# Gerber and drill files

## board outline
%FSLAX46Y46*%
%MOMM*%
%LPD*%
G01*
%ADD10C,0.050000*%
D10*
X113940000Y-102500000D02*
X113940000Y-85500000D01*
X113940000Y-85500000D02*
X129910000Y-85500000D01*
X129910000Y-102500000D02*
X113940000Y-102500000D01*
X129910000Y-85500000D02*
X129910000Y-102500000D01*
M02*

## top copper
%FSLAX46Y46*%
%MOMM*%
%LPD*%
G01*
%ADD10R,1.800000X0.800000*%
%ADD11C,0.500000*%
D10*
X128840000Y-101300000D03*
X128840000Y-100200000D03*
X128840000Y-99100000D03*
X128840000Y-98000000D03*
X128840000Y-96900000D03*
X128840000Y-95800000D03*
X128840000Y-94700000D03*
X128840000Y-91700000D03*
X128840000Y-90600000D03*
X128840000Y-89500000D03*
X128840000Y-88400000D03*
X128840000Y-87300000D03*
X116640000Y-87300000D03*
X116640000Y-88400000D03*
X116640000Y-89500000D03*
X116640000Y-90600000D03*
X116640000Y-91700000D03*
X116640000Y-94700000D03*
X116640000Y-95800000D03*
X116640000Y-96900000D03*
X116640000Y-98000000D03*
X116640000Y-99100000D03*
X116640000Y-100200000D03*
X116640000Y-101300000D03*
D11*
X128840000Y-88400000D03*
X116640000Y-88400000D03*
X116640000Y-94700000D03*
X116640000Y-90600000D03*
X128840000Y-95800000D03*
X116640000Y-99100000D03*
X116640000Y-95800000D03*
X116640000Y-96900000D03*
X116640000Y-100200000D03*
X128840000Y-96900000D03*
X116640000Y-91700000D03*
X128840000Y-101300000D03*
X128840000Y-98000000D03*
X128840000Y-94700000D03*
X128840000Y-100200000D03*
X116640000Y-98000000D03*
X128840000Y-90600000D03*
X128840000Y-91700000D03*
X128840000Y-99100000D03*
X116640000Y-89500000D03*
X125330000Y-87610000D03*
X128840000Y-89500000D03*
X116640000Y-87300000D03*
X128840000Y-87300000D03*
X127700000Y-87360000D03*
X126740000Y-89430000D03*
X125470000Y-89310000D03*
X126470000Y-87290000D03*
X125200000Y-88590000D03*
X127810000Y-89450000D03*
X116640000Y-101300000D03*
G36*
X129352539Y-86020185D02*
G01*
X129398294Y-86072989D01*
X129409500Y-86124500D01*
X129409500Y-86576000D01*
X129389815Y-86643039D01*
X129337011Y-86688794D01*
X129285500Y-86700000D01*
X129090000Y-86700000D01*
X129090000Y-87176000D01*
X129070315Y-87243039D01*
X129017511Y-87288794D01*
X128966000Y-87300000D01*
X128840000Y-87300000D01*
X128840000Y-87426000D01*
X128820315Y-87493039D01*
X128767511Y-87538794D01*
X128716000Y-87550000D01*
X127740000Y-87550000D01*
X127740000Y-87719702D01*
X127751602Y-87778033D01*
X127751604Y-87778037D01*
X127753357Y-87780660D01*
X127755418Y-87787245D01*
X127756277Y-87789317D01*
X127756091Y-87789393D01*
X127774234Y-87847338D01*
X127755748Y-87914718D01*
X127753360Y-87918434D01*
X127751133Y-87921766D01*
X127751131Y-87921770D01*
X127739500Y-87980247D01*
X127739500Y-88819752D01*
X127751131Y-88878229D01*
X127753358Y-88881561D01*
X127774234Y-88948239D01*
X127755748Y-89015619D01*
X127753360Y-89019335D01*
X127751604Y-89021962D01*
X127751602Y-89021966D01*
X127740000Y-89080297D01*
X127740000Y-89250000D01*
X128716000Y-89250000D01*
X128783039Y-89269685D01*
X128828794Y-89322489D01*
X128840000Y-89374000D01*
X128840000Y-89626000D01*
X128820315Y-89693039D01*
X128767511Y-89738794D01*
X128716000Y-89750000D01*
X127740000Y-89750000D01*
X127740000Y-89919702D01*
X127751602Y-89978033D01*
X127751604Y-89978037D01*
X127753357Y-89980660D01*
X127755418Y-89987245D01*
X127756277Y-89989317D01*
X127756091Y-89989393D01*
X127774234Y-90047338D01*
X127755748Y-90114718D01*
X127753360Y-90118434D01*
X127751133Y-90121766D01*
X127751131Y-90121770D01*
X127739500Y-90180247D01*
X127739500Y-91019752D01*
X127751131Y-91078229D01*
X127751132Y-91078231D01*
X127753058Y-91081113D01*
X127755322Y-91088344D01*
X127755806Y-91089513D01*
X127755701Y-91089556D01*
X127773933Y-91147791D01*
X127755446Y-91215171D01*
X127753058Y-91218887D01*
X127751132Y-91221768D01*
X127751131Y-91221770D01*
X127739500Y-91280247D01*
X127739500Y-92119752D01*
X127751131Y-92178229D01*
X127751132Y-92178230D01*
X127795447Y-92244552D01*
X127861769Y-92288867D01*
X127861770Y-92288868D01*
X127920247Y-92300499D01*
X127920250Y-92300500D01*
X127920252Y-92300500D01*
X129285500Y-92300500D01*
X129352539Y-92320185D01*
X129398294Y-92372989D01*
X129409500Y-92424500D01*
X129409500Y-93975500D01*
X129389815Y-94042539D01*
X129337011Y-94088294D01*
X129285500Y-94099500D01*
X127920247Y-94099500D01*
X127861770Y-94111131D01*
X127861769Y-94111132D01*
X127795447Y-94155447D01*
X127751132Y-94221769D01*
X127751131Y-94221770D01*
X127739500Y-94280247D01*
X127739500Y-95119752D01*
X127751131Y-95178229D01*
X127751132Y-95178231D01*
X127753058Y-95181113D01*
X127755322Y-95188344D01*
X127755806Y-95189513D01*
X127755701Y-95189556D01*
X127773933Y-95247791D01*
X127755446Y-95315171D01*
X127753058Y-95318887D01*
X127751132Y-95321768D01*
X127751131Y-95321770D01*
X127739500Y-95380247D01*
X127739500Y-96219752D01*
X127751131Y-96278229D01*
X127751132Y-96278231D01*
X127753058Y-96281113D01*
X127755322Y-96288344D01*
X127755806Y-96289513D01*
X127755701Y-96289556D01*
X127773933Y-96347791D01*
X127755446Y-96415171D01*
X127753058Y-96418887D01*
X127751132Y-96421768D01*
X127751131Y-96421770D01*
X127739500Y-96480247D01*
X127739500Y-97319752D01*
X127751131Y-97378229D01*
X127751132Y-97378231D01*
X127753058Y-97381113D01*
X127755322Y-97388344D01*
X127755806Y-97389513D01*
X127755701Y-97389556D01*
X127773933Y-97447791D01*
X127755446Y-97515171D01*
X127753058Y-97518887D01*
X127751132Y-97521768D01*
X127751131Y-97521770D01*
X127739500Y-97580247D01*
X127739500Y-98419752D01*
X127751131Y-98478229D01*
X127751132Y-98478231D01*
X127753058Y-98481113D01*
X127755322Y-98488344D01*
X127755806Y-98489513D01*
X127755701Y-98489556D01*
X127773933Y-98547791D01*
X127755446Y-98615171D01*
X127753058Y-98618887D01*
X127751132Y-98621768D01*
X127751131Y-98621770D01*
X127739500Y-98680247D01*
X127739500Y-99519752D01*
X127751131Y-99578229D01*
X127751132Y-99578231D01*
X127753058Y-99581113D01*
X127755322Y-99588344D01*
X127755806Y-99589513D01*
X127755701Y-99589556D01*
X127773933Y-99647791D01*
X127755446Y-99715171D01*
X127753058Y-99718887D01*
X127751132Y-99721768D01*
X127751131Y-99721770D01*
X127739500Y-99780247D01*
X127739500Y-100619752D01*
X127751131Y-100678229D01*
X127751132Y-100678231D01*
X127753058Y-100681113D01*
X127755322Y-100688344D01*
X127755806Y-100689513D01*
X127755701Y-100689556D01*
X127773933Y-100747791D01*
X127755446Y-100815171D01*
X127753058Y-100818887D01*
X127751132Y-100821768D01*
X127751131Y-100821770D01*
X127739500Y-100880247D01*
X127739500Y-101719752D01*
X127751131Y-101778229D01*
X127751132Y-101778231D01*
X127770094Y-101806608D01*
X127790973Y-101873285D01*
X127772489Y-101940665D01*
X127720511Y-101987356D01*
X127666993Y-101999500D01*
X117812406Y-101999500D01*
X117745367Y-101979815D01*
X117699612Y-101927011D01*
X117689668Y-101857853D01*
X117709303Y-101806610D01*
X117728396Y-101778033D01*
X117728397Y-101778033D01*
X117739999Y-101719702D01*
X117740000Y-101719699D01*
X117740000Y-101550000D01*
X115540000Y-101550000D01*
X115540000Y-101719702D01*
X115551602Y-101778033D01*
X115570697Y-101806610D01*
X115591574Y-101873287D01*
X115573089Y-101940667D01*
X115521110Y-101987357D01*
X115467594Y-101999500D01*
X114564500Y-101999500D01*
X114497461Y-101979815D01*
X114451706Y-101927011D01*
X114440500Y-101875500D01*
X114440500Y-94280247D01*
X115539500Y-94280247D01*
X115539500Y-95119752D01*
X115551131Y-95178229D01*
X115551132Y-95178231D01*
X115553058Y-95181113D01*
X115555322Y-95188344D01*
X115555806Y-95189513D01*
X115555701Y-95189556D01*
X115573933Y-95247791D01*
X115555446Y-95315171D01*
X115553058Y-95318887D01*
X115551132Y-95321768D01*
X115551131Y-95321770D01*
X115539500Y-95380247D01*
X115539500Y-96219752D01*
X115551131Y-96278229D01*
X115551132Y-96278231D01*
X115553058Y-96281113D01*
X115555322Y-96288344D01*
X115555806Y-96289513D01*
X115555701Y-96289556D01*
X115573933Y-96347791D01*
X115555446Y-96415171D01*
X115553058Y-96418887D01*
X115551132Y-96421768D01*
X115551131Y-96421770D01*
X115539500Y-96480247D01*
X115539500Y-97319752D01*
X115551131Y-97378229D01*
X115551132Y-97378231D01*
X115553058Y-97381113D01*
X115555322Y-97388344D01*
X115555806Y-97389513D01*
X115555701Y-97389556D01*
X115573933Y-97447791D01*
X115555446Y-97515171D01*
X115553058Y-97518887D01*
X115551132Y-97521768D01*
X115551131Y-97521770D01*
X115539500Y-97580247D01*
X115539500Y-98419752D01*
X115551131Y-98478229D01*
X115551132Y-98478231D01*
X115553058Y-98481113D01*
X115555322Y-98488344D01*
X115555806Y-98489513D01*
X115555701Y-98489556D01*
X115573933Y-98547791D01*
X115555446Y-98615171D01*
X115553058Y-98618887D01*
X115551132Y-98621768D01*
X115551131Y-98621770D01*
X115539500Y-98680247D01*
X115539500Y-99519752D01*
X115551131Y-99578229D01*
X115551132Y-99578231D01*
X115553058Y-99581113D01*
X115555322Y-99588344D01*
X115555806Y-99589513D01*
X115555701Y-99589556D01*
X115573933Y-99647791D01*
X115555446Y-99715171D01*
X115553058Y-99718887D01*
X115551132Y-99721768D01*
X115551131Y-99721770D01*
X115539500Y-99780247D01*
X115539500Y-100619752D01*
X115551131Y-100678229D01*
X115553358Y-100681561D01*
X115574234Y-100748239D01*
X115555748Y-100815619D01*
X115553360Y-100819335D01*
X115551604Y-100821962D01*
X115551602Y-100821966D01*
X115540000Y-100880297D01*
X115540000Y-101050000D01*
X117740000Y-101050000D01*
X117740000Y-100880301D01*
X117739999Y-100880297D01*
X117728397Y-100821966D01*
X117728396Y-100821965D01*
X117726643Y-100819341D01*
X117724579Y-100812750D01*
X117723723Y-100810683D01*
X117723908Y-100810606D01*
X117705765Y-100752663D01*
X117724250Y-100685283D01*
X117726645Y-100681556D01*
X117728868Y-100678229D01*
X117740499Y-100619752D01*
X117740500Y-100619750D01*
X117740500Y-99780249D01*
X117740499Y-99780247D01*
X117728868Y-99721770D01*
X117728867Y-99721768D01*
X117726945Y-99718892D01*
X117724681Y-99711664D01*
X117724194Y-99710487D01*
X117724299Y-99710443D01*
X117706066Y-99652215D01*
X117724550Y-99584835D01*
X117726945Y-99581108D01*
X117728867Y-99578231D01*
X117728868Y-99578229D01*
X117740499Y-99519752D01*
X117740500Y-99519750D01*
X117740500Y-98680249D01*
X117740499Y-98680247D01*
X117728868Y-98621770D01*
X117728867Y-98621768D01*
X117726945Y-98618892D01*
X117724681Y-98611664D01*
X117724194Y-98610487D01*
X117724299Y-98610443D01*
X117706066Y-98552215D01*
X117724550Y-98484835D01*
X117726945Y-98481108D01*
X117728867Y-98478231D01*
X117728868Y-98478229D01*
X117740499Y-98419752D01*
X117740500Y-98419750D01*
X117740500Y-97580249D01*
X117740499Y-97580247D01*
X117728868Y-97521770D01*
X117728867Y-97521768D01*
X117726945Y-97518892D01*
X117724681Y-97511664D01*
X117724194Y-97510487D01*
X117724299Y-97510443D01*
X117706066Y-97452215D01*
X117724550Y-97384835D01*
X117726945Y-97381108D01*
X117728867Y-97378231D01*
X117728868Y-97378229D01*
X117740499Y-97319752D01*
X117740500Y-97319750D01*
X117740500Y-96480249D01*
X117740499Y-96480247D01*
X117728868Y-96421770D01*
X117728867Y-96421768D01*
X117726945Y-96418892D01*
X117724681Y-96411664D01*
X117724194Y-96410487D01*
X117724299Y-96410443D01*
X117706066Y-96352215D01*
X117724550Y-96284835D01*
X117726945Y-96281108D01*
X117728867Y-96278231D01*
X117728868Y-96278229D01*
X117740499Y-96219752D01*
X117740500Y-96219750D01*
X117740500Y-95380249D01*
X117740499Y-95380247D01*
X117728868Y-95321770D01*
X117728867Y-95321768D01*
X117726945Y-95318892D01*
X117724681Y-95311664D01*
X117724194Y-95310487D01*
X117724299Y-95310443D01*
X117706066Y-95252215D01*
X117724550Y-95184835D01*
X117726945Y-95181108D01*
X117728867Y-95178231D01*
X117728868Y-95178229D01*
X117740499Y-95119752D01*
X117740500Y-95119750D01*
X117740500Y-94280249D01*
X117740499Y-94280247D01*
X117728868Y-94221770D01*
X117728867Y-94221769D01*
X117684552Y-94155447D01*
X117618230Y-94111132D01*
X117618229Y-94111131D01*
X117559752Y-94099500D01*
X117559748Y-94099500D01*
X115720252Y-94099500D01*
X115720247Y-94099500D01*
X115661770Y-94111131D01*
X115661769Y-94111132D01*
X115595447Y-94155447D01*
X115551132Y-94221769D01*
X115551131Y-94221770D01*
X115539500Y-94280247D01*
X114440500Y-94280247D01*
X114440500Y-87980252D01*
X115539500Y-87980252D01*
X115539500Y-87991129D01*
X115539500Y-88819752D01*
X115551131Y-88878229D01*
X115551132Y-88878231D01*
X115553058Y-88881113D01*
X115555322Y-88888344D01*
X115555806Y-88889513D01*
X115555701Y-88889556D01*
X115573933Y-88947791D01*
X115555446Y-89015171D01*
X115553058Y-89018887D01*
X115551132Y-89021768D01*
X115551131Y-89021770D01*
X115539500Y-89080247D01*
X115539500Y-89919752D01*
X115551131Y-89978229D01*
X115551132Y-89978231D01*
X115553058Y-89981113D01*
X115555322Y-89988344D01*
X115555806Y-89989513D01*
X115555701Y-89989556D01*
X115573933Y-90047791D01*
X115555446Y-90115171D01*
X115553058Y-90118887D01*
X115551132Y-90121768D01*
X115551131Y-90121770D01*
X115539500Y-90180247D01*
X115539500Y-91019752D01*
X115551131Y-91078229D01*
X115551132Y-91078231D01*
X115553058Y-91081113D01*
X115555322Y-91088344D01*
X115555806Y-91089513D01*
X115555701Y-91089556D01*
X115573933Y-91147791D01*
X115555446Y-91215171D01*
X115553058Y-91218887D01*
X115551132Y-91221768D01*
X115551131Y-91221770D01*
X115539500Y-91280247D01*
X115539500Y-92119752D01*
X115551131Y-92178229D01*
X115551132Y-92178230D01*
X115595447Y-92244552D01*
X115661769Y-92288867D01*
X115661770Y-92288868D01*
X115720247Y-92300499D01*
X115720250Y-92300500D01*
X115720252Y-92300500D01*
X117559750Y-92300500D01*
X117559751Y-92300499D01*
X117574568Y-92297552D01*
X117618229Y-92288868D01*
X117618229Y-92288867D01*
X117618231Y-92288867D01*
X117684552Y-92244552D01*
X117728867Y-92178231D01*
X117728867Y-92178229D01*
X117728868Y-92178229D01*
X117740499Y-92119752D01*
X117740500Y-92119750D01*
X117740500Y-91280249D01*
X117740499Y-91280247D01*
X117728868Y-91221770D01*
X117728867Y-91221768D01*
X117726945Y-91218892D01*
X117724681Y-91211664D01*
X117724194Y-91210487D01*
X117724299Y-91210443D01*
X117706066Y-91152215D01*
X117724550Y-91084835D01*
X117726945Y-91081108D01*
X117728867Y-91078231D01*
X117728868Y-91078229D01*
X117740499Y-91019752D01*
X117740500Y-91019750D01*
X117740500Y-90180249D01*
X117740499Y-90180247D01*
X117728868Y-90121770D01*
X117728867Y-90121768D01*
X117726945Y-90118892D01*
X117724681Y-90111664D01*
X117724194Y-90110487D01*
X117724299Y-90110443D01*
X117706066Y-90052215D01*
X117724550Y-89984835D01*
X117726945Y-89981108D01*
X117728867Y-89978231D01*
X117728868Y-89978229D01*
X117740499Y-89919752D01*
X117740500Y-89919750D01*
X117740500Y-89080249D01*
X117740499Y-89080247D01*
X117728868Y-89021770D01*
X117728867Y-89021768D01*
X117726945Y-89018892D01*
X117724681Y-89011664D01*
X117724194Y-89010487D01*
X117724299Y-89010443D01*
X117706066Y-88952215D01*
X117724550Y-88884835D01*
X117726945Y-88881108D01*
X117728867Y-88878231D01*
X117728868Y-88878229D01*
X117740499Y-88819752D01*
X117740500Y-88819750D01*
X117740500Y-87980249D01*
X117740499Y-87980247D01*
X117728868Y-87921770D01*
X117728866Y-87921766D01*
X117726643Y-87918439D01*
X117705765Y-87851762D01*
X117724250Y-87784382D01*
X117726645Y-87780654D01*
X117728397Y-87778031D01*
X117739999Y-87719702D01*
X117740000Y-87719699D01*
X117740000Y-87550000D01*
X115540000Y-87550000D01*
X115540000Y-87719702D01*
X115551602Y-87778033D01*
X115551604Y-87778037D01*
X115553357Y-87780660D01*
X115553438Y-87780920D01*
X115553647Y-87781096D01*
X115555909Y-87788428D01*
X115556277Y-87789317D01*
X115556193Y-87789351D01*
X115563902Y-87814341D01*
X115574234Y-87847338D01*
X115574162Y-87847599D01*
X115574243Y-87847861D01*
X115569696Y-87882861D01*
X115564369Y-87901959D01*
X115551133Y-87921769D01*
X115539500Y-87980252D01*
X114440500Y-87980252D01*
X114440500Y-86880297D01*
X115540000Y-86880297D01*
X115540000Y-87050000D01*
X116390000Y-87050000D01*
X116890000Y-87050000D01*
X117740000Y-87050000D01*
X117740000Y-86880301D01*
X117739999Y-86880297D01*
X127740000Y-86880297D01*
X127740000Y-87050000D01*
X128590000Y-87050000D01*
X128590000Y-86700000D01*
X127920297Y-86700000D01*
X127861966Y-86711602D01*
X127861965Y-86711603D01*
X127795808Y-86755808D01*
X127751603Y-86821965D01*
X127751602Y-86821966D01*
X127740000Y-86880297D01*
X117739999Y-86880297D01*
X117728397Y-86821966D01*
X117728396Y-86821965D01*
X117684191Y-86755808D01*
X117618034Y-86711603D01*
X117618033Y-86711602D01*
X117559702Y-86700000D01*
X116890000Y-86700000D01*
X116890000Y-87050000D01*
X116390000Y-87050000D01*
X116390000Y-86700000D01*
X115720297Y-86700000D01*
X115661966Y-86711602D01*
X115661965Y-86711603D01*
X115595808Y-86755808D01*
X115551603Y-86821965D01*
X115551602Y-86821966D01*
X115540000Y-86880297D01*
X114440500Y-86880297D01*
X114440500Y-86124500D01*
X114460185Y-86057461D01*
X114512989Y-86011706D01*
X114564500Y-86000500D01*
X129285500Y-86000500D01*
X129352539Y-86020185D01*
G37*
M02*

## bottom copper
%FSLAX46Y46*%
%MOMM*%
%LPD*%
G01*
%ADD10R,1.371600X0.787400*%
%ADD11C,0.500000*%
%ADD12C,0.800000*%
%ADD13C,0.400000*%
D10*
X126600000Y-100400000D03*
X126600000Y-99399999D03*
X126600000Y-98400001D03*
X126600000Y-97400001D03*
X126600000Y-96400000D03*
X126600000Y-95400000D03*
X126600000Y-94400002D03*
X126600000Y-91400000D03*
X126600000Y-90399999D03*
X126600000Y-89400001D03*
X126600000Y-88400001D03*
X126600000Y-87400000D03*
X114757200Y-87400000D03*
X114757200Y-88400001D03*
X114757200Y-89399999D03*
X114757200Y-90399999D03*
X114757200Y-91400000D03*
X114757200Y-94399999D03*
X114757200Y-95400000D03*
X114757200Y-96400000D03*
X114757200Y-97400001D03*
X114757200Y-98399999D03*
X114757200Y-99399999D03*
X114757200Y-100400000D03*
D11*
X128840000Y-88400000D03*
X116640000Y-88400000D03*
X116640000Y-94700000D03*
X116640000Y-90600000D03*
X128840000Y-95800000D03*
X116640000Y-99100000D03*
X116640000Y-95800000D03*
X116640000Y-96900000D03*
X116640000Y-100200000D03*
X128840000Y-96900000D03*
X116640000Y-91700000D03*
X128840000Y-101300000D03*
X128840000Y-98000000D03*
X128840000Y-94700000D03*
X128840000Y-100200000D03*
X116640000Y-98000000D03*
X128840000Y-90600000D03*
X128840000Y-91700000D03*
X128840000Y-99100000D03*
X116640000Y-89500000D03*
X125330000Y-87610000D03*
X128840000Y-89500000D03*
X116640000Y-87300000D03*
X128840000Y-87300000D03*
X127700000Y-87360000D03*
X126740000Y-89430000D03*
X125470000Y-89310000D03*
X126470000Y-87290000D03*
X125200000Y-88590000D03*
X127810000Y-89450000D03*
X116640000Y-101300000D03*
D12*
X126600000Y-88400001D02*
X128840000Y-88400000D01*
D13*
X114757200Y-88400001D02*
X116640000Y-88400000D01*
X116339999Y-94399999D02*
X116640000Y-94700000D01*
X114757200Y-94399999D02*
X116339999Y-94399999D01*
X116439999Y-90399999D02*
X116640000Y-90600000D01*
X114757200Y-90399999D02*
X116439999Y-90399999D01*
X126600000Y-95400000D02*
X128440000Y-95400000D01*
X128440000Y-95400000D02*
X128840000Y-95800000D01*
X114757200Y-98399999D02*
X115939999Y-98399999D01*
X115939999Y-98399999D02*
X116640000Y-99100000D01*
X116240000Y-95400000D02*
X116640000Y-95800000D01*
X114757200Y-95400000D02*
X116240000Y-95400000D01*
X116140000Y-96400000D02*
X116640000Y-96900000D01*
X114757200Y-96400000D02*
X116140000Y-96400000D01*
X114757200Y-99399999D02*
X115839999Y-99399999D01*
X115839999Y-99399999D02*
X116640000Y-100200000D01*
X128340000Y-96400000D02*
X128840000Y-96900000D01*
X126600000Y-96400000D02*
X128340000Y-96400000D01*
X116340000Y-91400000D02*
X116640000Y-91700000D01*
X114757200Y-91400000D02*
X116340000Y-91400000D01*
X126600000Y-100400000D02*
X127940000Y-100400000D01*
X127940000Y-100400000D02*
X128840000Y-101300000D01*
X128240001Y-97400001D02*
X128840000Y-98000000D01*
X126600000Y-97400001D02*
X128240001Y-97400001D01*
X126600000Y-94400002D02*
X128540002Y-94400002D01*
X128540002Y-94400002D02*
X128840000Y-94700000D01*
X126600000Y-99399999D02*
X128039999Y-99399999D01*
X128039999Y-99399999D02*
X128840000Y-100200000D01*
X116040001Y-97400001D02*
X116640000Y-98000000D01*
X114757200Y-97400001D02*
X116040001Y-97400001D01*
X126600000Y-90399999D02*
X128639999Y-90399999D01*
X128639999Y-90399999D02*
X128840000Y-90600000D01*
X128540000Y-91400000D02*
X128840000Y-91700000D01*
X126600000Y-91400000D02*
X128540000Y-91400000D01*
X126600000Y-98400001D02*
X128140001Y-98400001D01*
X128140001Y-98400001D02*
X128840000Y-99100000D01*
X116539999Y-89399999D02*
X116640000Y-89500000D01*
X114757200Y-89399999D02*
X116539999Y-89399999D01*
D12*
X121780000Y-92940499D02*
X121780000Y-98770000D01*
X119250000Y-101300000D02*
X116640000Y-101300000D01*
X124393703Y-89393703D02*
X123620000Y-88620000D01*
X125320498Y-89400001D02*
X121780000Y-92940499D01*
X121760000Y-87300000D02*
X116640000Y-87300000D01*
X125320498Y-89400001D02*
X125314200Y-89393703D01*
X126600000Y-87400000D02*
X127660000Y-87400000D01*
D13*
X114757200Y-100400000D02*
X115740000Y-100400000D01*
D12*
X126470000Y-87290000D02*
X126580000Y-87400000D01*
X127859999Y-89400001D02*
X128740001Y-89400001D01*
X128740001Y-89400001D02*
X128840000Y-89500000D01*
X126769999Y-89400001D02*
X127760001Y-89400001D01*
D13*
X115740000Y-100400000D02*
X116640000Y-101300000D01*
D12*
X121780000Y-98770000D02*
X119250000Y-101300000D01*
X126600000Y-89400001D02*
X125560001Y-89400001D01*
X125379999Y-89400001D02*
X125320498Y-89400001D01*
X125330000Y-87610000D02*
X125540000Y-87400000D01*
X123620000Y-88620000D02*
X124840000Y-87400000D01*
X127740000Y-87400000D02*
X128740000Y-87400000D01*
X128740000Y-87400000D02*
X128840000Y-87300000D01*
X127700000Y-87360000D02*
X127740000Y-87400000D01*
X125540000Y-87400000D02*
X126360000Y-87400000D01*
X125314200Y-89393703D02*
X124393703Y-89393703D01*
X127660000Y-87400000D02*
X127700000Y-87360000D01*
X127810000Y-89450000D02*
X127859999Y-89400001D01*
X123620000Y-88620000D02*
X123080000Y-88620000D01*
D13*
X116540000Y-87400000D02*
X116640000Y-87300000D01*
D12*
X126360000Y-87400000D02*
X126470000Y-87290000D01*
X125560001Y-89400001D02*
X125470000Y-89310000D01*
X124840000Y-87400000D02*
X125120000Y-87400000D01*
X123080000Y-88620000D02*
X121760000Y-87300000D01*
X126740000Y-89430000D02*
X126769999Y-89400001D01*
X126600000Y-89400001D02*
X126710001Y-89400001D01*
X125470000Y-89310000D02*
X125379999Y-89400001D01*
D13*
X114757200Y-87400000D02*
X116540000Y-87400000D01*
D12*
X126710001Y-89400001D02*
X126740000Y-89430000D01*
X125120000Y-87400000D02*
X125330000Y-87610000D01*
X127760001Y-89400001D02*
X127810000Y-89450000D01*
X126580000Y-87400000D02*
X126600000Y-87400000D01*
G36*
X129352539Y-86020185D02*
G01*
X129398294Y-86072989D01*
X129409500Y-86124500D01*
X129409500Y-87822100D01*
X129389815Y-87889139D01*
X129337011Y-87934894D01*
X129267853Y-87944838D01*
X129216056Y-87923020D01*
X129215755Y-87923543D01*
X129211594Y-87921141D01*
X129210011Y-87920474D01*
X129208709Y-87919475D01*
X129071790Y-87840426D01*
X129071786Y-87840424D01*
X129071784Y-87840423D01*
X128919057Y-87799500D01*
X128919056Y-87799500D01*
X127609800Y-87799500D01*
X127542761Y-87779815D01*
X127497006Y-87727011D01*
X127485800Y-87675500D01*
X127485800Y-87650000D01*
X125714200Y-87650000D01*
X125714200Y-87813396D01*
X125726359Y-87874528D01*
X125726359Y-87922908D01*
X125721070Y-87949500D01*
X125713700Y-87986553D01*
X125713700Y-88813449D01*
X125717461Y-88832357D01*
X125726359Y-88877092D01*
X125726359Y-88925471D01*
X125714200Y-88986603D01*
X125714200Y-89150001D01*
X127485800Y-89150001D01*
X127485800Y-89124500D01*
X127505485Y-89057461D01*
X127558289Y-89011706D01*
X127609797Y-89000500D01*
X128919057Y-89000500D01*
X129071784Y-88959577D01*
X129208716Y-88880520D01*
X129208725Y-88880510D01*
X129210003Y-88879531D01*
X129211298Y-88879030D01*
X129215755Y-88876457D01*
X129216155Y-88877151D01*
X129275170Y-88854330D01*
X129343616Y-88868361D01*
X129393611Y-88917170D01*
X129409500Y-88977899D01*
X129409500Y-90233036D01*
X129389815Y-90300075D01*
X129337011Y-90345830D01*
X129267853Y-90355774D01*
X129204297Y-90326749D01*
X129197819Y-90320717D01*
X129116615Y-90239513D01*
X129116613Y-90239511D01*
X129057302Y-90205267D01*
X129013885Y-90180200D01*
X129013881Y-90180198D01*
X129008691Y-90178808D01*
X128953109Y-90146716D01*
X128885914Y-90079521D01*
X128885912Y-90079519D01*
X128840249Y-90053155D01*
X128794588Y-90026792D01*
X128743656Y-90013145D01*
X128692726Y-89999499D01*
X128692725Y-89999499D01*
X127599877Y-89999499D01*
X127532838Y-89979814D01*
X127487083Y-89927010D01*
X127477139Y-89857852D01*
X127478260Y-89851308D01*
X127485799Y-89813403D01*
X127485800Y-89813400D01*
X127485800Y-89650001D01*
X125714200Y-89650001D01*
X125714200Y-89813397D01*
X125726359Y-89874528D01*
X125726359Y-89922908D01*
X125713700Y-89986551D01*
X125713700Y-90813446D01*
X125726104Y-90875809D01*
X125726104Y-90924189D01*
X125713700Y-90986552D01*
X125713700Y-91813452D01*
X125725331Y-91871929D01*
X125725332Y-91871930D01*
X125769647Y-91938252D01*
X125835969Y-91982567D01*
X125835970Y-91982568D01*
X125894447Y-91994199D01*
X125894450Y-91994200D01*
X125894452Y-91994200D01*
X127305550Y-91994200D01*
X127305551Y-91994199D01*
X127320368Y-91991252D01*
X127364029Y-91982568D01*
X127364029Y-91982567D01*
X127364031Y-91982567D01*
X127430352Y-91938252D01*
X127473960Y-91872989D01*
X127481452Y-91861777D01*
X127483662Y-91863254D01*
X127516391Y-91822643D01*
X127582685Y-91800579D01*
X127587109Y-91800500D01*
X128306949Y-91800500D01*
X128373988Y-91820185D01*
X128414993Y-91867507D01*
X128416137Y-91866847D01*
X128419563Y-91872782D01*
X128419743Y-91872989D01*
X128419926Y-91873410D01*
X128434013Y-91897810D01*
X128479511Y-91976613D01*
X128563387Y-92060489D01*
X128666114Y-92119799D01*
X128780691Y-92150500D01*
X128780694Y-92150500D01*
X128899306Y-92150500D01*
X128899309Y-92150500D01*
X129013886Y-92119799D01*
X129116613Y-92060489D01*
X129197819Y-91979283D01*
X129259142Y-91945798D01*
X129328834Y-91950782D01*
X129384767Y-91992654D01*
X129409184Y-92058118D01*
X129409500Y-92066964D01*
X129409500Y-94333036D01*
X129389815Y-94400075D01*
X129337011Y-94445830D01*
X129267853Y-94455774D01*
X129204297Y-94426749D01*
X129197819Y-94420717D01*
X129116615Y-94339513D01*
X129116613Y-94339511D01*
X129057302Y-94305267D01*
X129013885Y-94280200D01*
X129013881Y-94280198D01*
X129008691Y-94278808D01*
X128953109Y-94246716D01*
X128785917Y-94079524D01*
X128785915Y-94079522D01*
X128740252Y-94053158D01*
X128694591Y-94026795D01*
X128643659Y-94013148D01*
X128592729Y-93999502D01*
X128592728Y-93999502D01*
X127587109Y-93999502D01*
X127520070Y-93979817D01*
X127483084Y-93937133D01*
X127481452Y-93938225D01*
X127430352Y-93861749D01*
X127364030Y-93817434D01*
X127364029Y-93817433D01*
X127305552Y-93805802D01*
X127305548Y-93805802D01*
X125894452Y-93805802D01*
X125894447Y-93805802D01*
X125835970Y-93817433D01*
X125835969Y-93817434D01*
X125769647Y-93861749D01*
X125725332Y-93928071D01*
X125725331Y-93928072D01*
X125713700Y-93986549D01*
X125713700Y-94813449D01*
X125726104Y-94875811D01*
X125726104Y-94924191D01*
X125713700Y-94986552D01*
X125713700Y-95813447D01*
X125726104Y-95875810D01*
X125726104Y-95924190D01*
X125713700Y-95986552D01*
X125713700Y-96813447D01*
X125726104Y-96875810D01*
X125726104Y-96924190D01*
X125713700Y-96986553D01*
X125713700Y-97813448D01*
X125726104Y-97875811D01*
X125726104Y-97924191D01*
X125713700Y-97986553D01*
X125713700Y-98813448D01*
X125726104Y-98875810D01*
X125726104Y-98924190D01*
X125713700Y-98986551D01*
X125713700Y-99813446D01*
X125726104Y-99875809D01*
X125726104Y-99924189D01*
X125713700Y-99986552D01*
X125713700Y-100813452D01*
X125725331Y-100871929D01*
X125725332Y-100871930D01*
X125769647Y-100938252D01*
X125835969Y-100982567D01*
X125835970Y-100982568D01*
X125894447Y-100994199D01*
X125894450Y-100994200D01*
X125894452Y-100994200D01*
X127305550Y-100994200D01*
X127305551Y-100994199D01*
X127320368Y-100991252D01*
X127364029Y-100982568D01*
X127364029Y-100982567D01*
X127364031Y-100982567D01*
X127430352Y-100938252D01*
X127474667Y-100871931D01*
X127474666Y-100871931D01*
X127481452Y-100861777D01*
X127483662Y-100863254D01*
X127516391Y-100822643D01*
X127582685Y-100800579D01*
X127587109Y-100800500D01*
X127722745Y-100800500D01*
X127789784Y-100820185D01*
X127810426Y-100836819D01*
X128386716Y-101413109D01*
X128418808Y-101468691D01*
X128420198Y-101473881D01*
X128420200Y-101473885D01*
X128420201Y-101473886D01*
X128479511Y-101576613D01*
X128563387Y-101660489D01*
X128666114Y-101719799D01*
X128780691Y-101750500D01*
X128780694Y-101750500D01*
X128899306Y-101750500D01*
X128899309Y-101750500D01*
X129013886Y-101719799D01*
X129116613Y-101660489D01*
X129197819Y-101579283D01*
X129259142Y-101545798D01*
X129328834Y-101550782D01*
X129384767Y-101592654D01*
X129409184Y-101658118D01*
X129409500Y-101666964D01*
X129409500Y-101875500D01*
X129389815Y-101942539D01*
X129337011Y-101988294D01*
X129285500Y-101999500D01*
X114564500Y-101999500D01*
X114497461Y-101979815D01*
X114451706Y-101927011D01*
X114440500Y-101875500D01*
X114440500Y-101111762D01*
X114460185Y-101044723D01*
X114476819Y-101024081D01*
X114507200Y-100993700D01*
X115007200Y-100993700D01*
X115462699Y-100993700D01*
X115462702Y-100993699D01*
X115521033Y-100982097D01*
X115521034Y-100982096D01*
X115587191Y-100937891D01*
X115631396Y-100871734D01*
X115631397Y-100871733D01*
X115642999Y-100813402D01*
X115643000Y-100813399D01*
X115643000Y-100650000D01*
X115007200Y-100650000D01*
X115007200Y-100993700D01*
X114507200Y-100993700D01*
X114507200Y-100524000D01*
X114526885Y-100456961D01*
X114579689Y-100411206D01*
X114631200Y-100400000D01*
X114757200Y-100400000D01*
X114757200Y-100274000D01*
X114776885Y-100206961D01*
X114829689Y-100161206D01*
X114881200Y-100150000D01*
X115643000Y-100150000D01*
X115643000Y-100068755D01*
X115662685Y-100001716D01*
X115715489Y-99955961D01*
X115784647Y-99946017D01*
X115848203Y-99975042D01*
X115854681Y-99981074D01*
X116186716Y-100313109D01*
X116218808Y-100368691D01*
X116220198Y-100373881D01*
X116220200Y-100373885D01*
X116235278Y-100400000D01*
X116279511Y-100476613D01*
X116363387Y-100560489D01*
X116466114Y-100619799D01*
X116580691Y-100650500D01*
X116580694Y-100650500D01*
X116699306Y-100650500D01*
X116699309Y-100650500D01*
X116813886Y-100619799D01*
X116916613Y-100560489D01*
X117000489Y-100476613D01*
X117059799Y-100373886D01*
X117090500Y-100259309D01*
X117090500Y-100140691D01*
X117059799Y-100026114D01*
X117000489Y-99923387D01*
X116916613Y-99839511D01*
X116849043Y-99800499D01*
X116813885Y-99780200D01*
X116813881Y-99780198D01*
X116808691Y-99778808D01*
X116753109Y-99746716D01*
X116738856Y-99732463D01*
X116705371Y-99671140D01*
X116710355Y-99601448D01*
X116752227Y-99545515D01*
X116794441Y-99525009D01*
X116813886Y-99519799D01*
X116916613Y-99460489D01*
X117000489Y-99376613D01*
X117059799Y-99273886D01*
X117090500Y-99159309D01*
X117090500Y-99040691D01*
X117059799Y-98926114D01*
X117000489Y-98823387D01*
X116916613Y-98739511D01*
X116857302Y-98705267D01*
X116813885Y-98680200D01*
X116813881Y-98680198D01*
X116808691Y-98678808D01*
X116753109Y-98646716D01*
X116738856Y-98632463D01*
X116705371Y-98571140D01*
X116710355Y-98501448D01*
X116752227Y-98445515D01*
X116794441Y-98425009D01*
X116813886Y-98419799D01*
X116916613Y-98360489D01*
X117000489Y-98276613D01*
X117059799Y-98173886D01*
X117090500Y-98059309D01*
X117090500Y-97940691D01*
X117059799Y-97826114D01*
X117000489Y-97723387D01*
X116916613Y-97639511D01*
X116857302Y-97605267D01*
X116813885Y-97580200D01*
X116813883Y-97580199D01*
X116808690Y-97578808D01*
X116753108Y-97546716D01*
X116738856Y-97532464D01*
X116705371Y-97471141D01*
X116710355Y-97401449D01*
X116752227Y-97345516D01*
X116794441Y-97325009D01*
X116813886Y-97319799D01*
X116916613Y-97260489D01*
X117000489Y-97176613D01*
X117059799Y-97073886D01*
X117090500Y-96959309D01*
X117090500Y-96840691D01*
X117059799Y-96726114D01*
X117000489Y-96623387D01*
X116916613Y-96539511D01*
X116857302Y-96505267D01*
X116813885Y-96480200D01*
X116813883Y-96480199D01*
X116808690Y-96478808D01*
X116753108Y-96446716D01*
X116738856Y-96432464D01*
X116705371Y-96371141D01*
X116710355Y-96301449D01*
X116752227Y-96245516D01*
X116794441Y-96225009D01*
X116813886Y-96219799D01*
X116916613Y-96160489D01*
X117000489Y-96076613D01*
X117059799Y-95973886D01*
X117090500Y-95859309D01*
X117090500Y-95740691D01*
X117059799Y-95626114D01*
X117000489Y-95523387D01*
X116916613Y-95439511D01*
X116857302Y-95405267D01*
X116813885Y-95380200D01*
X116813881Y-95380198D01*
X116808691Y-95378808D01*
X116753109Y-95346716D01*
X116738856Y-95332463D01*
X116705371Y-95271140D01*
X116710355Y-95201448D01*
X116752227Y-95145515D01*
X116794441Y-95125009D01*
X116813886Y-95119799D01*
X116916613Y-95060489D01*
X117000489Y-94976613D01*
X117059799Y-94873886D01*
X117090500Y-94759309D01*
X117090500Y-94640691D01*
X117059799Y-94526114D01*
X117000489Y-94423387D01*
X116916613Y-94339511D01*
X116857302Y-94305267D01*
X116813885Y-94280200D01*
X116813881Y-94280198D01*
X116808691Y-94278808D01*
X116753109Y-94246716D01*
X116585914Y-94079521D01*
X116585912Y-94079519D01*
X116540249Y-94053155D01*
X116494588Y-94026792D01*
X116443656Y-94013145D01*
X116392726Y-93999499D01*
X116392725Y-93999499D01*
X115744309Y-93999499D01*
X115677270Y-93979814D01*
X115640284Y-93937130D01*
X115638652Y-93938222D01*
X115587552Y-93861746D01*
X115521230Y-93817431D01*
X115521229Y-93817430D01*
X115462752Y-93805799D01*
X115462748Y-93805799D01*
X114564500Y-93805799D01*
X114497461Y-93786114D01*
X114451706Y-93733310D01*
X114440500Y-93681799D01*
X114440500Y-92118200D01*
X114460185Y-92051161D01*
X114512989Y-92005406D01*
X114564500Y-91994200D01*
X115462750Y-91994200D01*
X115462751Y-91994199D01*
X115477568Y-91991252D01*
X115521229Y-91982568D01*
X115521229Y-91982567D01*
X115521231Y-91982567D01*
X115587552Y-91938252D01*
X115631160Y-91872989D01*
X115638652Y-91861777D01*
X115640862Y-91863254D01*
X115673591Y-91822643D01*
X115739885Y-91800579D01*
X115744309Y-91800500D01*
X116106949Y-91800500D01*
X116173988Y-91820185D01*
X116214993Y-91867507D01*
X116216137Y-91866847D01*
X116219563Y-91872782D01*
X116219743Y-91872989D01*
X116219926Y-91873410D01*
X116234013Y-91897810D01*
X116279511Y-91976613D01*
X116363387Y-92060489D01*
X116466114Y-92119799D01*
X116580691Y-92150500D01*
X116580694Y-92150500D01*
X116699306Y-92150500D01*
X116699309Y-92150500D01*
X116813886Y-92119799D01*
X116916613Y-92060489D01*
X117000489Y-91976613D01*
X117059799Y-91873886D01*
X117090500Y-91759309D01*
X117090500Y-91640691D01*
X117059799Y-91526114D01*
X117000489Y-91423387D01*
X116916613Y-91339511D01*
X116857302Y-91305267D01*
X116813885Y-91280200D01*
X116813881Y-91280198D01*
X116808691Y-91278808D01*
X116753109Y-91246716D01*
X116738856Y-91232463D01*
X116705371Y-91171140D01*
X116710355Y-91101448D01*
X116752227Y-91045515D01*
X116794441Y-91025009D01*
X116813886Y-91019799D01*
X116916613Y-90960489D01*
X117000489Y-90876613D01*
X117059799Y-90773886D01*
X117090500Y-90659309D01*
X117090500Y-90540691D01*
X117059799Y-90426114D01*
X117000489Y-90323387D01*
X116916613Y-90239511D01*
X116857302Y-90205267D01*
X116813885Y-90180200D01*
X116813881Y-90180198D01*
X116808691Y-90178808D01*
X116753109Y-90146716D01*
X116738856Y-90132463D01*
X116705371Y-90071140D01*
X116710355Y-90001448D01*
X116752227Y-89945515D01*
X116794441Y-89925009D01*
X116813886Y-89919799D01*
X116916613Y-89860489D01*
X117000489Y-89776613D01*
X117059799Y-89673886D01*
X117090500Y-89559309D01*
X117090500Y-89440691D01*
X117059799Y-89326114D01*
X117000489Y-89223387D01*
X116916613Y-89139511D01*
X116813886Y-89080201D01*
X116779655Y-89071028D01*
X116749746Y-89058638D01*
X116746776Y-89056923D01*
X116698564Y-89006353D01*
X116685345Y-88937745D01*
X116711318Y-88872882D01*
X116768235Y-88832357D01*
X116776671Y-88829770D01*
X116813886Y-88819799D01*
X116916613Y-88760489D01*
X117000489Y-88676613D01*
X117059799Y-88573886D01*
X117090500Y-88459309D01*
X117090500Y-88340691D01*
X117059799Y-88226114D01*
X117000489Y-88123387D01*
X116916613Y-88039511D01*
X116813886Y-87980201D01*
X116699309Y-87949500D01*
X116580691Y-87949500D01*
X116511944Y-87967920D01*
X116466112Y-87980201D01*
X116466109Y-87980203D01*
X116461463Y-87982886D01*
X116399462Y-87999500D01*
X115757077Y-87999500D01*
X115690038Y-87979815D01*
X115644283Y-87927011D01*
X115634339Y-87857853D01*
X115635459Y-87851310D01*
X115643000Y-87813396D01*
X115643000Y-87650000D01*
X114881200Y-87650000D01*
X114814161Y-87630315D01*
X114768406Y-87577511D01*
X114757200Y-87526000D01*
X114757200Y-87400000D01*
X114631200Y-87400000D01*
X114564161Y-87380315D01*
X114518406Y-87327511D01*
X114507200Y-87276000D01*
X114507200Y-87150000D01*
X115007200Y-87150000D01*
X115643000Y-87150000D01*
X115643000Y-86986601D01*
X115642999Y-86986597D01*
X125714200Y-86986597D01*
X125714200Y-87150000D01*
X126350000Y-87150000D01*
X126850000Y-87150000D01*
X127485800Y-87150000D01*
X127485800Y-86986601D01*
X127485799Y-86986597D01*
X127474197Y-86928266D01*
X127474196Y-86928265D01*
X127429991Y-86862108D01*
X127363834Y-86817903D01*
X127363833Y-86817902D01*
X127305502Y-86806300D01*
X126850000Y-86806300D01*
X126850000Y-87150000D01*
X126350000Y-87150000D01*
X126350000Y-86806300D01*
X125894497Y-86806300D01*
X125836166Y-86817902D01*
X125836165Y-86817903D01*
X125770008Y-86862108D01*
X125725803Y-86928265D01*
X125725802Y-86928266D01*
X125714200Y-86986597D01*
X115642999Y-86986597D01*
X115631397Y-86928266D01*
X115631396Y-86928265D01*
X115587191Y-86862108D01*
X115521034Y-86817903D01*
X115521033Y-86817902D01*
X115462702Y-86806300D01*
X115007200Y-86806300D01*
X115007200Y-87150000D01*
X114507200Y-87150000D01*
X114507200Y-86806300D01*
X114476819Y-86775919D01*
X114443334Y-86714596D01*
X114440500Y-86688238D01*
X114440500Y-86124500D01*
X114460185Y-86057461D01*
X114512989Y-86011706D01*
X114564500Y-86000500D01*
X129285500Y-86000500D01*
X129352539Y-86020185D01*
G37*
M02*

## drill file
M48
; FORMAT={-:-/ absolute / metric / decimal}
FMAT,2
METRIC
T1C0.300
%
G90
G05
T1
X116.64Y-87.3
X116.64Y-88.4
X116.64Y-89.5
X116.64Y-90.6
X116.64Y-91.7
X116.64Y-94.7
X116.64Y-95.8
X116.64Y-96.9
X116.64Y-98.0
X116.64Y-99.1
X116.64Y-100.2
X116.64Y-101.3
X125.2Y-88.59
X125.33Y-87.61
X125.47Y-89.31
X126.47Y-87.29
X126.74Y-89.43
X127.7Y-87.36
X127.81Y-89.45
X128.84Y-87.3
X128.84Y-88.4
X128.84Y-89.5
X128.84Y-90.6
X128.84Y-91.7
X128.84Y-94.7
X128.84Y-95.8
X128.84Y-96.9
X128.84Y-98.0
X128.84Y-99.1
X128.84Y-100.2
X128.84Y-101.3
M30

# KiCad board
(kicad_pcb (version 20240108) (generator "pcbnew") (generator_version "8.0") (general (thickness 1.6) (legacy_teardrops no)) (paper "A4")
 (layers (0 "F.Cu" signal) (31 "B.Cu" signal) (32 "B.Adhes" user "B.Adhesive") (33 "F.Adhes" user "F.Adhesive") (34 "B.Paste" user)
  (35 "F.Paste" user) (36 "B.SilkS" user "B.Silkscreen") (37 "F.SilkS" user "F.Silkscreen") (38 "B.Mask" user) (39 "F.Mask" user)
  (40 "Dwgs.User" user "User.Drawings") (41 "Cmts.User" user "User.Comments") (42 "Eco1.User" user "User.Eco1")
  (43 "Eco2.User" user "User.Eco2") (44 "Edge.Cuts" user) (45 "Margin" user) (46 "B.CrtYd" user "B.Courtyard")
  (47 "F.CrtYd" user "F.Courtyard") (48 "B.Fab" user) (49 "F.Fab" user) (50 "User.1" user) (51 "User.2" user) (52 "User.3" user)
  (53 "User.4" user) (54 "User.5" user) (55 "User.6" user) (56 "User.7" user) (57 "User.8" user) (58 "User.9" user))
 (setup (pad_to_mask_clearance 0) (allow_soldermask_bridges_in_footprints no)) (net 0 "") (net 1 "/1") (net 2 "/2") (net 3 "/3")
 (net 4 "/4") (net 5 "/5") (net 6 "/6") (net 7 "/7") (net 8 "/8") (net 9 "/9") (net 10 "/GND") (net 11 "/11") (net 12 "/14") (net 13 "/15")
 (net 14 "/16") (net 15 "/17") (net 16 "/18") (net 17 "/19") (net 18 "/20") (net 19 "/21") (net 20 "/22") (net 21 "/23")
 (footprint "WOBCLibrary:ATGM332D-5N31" (layer "F.Cu") (at 122.74 93.7)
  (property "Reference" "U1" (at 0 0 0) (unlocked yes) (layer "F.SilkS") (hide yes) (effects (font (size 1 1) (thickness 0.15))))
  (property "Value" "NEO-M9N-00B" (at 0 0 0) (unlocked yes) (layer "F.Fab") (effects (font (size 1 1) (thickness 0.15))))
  (pad "1" smd rect (at 6.1 7.6) (size 1.8 0.8) (layers "F.Cu" "F.Paste" "F.Mask") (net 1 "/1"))
  (pad "2" smd rect (at 6.1 6.5) (size 1.8 0.8) (layers "F.Cu" "F.Paste" "F.Mask") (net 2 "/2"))
  (pad "3" smd rect (at 6.1 5.4) (size 1.8 0.8) (layers "F.Cu" "F.Paste" "F.Mask") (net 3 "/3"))
  (pad "4" smd rect (at 6.1 4.3) (size 1.8 0.8) (layers "F.Cu" "F.Paste" "F.Mask") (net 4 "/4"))
  (pad "5" smd rect (at 6.1 3.2) (size 1.8 0.8) (layers "F.Cu" "F.Paste" "F.Mask") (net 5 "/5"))
  (pad "6" smd rect (at 6.1 2.1) (size 1.8 0.8) (layers "F.Cu" "F.Paste" "F.Mask") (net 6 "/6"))
  (pad "7" smd rect (at 6.1 1) (size 1.8 0.8) (layers "F.Cu" "F.Paste" "F.Mask") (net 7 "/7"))
  (pad "8" smd rect (at 6.1 -2) (size 1.8 0.8) (layers "F.Cu" "F.Paste" "F.Mask") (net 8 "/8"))
  (pad "9" smd rect (at 6.1 -3.1) (size 1.8 0.8) (layers "F.Cu" "F.Paste" "F.Mask") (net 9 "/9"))
  (pad "10" smd rect (at 6.1 -4.2) (size 1.8 0.8) (layers "F.Cu" "F.Paste" "F.Mask") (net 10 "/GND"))
  (pad "11" smd rect (at 6.1 -5.3) (size 1.8 0.8) (layers "F.Cu" "F.Paste" "F.Mask") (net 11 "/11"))
  (pad "12" smd rect (at 6.1 -6.4) (size 1.8 0.8) (layers "F.Cu" "F.Paste" "F.Mask") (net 10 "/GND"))
  (pad "13" smd rect (at -6.1 -6.4) (size 1.8 0.8) (layers "F.Cu" "F.Paste" "F.Mask") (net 10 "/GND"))
  (pad "14" smd rect (at -6.1 -5.3) (size 1.8 0.8) (layers "F.Cu" "F.Paste" "F.Mask") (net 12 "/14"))
  (pad "15" smd rect (at -6.1 -4.2) (size 1.8 0.8) (layers "F.Cu" "F.Paste" "F.Mask") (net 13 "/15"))
  (pad "16" smd rect (at -6.1 -3.1) (size 1.8 0.8) (layers "F.Cu" "F.Paste" "F.Mask") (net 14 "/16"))
  (pad "17" smd rect (at -6.1 -2) (size 1.8 0.8) (layers "F.Cu" "F.Paste" "F.Mask") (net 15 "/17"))
  (pad "18" smd rect (at -6.1 1) (size 1.8 0.8) (layers "F.Cu" "F.Paste" "F.Mask") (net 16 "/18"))
  (pad "19" smd rect (at -6.1 2.1) (size 1.8 0.8) (layers "F.Cu" "F.Paste" "F.Mask") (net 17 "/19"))
  (pad "20" smd rect (at -6.1 3.2) (size 1.8 0.8) (layers "F.Cu" "F.Paste" "F.Mask") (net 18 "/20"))
  (pad "21" smd rect (at -6.1 4.3) (size 1.8 0.8) (layers "F.Cu" "F.Paste" "F.Mask") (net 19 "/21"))
  (pad "22" smd rect (at -6.1 5.4) (size 1.8 0.8) (layers "F.Cu" "F.Paste" "F.Mask") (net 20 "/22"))
  (pad "23" smd rect (at -6.1 6.5) (size 1.8 0.8) (layers "F.Cu" "F.Paste" "F.Mask") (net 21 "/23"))
  (pad "24" smd rect (at -6.1 7.6) (size 1.8 0.8) (layers "F.Cu" "F.Paste" "F.Mask") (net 10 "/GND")))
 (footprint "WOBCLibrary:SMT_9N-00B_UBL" (layer "B.Cu") (at 120.6786 93.9 180)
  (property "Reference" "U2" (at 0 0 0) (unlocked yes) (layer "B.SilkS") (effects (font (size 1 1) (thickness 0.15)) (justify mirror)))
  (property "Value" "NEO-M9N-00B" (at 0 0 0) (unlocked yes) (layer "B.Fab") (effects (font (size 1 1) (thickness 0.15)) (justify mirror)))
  (pad "1" smd rect (at -5.9214 -6.5 180) (size 1.3716 0.7874) (layers "B.Cu" "B.Paste" "B.Mask") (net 1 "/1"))
  (pad "2" smd rect (at -5.9214 -5.499999 180) (size 1.3716 0.7874) (layers "B.Cu" "B.Paste" "B.Mask") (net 2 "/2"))
  (pad "3" smd rect (at -5.9214 -4.500001 180) (size 1.3716 0.7874) (layers "B.Cu" "B.Paste" "B.Mask") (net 3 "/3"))
  (pad "4" smd rect (at -5.9214 -3.500001 180) (size 1.3716 0.7874) (layers "B.Cu" "B.Paste" "B.Mask") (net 4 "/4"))
  (pad "5" smd rect (at -5.9214 -2.5 180) (size 1.3716 0.7874) (layers "B.Cu" "B.Paste" "B.Mask") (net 5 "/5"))
  (pad "6" smd rect (at -5.9214 -1.5 180) (size 1.3716 0.7874) (layers "B.Cu" "B.Paste" "B.Mask") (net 6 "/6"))
  (pad "7" smd rect (at -5.9214 -0.500002 180) (size 1.3716 0.7874) (layers "B.Cu" "B.Paste" "B.Mask") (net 7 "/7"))
  (pad "8" smd rect (at -5.9214 2.5 180) (size 1.3716 0.7874) (layers "B.Cu" "B.Paste" "B.Mask") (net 8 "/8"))
  (pad "9" smd rect (at -5.9214 3.500001 180) (size 1.3716 0.7874) (layers "B.Cu" "B.Paste" "B.Mask") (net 9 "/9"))
  (pad "10" smd rect (at -5.9214 4.499999 180) (size 1.3716 0.7874) (layers "B.Cu" "B.Paste" "B.Mask") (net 10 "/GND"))
  (pad "11" smd rect (at -5.9214 5.499999 180) (size 1.3716 0.7874) (layers "B.Cu" "B.Paste" "B.Mask") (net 11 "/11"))
  (pad "12" smd rect (at -5.9214 6.5 180) (size 1.3716 0.7874) (layers "B.Cu" "B.Paste" "B.Mask") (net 10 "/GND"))
  (pad "13" smd rect (at 5.9214 6.5 180) (size 1.3716 0.7874) (layers "B.Cu" "B.Paste" "B.Mask") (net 10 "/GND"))
  (pad "14" smd rect (at 5.9214 5.499999 180) (size 1.3716 0.7874) (layers "B.Cu" "B.Paste" "B.Mask") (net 12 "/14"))
  (pad "15" smd rect (at 5.9214 4.500001 180) (size 1.3716 0.7874) (layers "B.Cu" "B.Paste" "B.Mask") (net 13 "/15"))
  (pad "16" smd rect (at 5.9214 3.500001 180) (size 1.3716 0.7874) (layers "B.Cu" "B.Paste" "B.Mask") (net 14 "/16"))
  (pad "17" smd rect (at 5.9214 2.5 180) (size 1.3716 0.7874) (layers "B.Cu" "B.Paste" "B.Mask") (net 15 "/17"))
  (pad "18" smd rect (at 5.9214 -0.499999 180) (size 1.3716 0.7874) (layers "B.Cu" "B.Paste" "B.Mask") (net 16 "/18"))
  (pad "19" smd rect (at 5.9214 -1.5 180) (size 1.3716 0.7874) (layers "B.Cu" "B.Paste" "B.Mask") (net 17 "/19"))
  (pad "20" smd rect (at 5.9214 -2.5 180) (size 1.3716 0.7874) (layers "B.Cu" "B.Paste" "B.Mask") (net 18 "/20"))
  (pad "21" smd rect (at 5.9214 -3.500001 180) (size 1.3716 0.7874) (layers "B.Cu" "B.Paste" "B.Mask") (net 19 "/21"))
  (pad "22" smd rect (at 5.9214 -4.499999 180) (size 1.3716 0.7874) (layers "B.Cu" "B.Paste" "B.Mask") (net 20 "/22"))
  (pad "23" smd rect (at 5.9214 -5.499999 180) (size 1.3716 0.7874) (layers "B.Cu" "B.Paste" "B.Mask") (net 21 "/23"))
  (pad "24" smd rect (at 5.9214 -6.5 180) (size 1.3716 0.7874) (layers "B.Cu" "B.Paste" "B.Mask") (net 10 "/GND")))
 (gr_line (start 113.94 102.5) (end 113.94 85.5) (stroke (width 0.05) (type default)) (layer "Edge.Cuts"))
 (gr_line (start 113.94 85.5) (end 129.91 85.5) (stroke (width 0.05) (type default)) (layer "Edge.Cuts"))
 (gr_line (start 129.91 102.5) (end 113.94 102.5) (stroke (width 0.05) (type default)) (layer "Edge.Cuts"))
 (gr_line (start 129.91 85.5) (end 129.91 102.5) (stroke (width 0.05) (type default)) (layer "Edge.Cuts"))
 (via (at 128.84 88.4) (size 0.5) (drill 0.3) (layers "F.Cu" "B.Cu") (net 11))
 (segment (start 126.6 88.400001) (end 128.84 88.4) (width 0.8) (layer "B.Cu") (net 11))
 (via (at 116.64 88.4) (size 0.5) (drill 0.3) (layers "F.Cu" "B.Cu") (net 12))
 (segment (start 114.7572 88.400001) (end 116.64 88.4) (width 0.4) (layer "B.Cu") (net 12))
 (via (at 116.64 94.7) (size 0.5) (drill 0.3) (layers "F.Cu" "B.Cu") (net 16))
 (segment (start 116.339999 94.399999) (end 116.64 94.7) (width 0.4) (layer "B.Cu") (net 16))
 (segment (start 114.7572 94.399999) (end 116.339999 94.399999) (width 0.4) (layer "B.Cu") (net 16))
 (via (at 116.64 90.6) (size 0.5) (drill 0.3) (layers "F.Cu" "B.Cu") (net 14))
 (segment (start 116.439999 90.399999) (end 116.64 90.6) (width 0.4) (layer "B.Cu") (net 14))
 (segment (start 114.7572 90.399999) (end 116.439999 90.399999) (width 0.4) (layer "B.Cu") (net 14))
 (via (at 128.84 95.8) (size 0.5) (drill 0.3) (layers "F.Cu" "B.Cu") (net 6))
 (segment (start 126.6 95.4) (end 128.44 95.4) (width 0.4) (layer "B.Cu") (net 6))
 (segment (start 128.44 95.4) (end 128.84 95.8) (width 0.4) (layer "B.Cu") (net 6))
 (via (at 116.64 99.1) (size 0.5) (drill 0.3) (layers "F.Cu" "B.Cu") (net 20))
 (segment (start 114.7572 98.399999) (end 115.939999 98.399999) (width 0.4) (layer "B.Cu") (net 20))
 (segment (start 115.939999 98.399999) (end 116.64 99.1) (width 0.4) (layer "B.Cu") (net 20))
 (via (at 116.64 95.8) (size 0.5) (drill 0.3) (layers "F.Cu" "B.Cu") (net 17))
 (segment (start 116.24 95.4) (end 116.64 95.8) (width 0.4) (layer "B.Cu") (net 17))
 (segment (start 114.7572 95.4) (end 116.24 95.4) (width 0.4) (layer "B.Cu") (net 17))
 (via (at 116.64 96.9) (size 0.5) (drill 0.3) (layers "F.Cu" "B.Cu") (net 18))
 (segment (start 116.14 96.4) (end 116.64 96.9) (width 0.4) (layer "B.Cu") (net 18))
 (segment (start 114.7572 96.4) (end 116.14 96.4) (width 0.4) (layer "B.Cu") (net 18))
 (via (at 116.64 100.2) (size 0.5) (drill 0.3) (layers "F.Cu" "B.Cu") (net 21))
 (segment (start 114.7572 99.399999) (end 115.839999 99.399999) (width 0.4) (layer "B.Cu") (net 21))
 (segment (start 115.839999 99.399999) (end 116.64 100.2) (width 0.4) (layer "B.Cu") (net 21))
 (via (at 128.84 96.9) (size 0.5) (drill 0.3) (layers "F.Cu" "B.Cu") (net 5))
 (segment (start 128.34 96.4) (end 128.84 96.9) (width 0.4) (layer "B.Cu") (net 5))
 (segment (start 126.6 96.4) (end 128.34 96.4) (width 0.4) (layer "B.Cu") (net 5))
 (via (at 116.64 91.7) (size 0.5) (drill 0.3) (layers "F.Cu" "B.Cu") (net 15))
 (segment (start 116.34 91.4) (end 116.64 91.7) (width 0.4) (layer "B.Cu") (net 15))
 (segment (start 114.7572 91.4) (end 116.34 91.4) (width 0.4) (layer "B.Cu") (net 15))
 (via (at 128.84 101.3) (size 0.5) (drill 0.3) (layers "F.Cu" "B.Cu") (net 1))
 (segment (start 126.6 100.4) (end 127.94 100.4) (width 0.4) (layer "B.Cu") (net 1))
 (segment (start 127.94 100.4) (end 128.84 101.3) (width 0.4) (layer "B.Cu") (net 1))
 (via (at 128.84 98) (size 0.5) (drill 0.3) (layers "F.Cu" "B.Cu") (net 4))
 (segment (start 128.240001 97.400001) (end 128.84 98) (width 0.4) (layer "B.Cu") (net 4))
 (segment (start 126.6 97.400001) (end 128.240001 97.400001) (width 0.4) (layer "B.Cu") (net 4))
 (via (at 128.84 94.7) (size 0.5) (drill 0.3) (layers "F.Cu" "B.Cu") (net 7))
 (segment (start 126.6 94.400002) (end 128.540002 94.400002) (width 0.4) (layer "B.Cu") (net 7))
 (segment (start 128.540002 94.400002) (end 128.84 94.7) (width 0.4) (layer "B.Cu") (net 7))
 (via (at 128.84 100.2) (size 0.5) (drill 0.3) (layers "F.Cu" "B.Cu") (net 2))
 (segment (start 126.6 99.399999) (end 128.039999 99.399999) (width 0.4) (layer "B.Cu") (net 2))
 (segment (start 128.039999 99.399999) (end 128.84 100.2) (width 0.4) (layer "B.Cu") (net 2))
 (via (at 116.64 98) (size 0.5) (drill 0.3) (layers "F.Cu" "B.Cu") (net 19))
 (segment (start 116.040001 97.400001) (end 116.64 98) (width 0.4) (layer "B.Cu") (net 19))
 (segment (start 114.7572 97.400001) (end 116.040001 97.400001) (width 0.4) (layer "B.Cu") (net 19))
 (via (at 128.84 90.6) (size 0.5) (drill 0.3) (layers "F.Cu" "B.Cu") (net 9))
 (segment (start 126.6 90.399999) (end 128.639999 90.399999) (width 0.4) (layer "B.Cu") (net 9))
 (segment (start 128.639999 90.399999) (end 128.84 90.6) (width 0.4) (layer "B.Cu") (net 9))
 (via (at 128.84 91.7) (size 0.5) (drill 0.3) (layers "F.Cu" "B.Cu") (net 8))
 (segment (start 128.54 91.4) (end 128.84 91.7) (width 0.4) (layer "B.Cu") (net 8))
 (segment (start 126.6 91.4) (end 128.54 91.4) (width 0.4) (layer "B.Cu") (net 8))
 (via (at 128.84 99.1) (size 0.5) (drill 0.3) (layers "F.Cu" "B.Cu") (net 3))
 (segment (start 126.6 98.400001) (end 128.140001 98.400001) (width 0.4) (layer "B.Cu") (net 3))
 (segment (start 128.140001 98.400001) (end 128.84 99.1) (width 0.4) (layer "B.Cu") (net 3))
 (via (at 116.64 89.5) (size 0.5) (drill 0.3) (layers "F.Cu" "B.Cu") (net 13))
 (segment (start 116.539999 89.399999) (end 116.64 89.5) (width 0.4) (layer "B.Cu") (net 13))
 (segment (start 114.7572 89.399999) (end 116.539999 89.399999) (width 0.4) (layer "B.Cu") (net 13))
 (via (at 125.33 87.61) (size 0.5) (drill 0.3) (layers "F.Cu" "B.Cu") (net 10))
 (via (at 128.84 89.5) (size 0.5) (drill 0.3) (layers "F.Cu" "B.Cu") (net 10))
 (via (at 116.64 87.3) (size 0.5) (drill 0.3) (layers "F.Cu" "B.Cu") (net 10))
 (via (at 128.84 87.3) (size 0.5) (drill 0.3) (layers "F.Cu" "B.Cu") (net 10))
 (via (at 127.7 87.36) (size 0.5) (drill 0.3) (layers "F.Cu" "B.Cu") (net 10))
 (via (at 126.74 89.43) (size 0.5) (drill 0.3) (layers "F.Cu" "B.Cu") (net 10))
 (via (at 125.47 89.31) (size 0.5) (drill 0.3) (layers "F.Cu" "B.Cu") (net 10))
 (via (at 126.47 87.29) (size 0.5) (drill 0.3) (layers "F.Cu" "B.Cu") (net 10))
 (via (at 125.2 88.59) (size 0.5) (drill 0.3) (layers "F.Cu" "B.Cu") (free yes) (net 10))
 (via (at 127.81 89.45) (size 0.5) (drill 0.3) (layers "F.Cu" "B.Cu") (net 10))
 (via (at 116.64 101.3) (size 0.5) (drill 0.3) (layers "F.Cu" "B.Cu") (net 10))
 (segment (start 121.78 92.940499) (end 121.78 98.77) (width 0.8) (layer "B.Cu") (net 10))
 (segment (start 119.25 101.3) (end 116.64 101.3) (width 0.8) (layer "B.Cu") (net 10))
 (segment (start 124.393703 89.393703) (end 123.62 88.62) (width 0.8) (layer "B.Cu") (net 10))
 (segment (start 125.320498 89.400001) (end 121.78 92.940499) (width 0.8) (layer "B.Cu") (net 10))
 (segment (start 121.76 87.3) (end 116.64 87.3) (width 0.8) (layer "B.Cu") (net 10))
 (segment (start 125.320498 89.400001) (end 125.3142 89.393703) (width 0.8) (layer "B.Cu") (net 10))
 (segment (start 126.6 87.4) (end 127.66 87.4) (width 0.8) (layer "B.Cu") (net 10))
 (segment (start 114.7572 100.4) (end 115.74 100.4) (width 0.4) (layer "B.Cu") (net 10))
 (segment (start 126.47 87.29) (end 126.58 87.4) (width 0.8) (layer "B.Cu") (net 10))
 (segment (start 127.859999 89.400001) (end 128.740001 89.400001) (width 0.8) (layer "B.Cu") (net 10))
 (segment (start 128.740001 89.400001) (end 128.84 89.5) (width 0.8) (layer "B.Cu") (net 10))
 (segment (start 126.769999 89.400001) (end 127.760001 89.400001) (width 0.8) (layer "B.Cu") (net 10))
 (segment (start 115.74 100.4) (end 116.64 101.3) (width 0.4) (layer "B.Cu") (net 10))
 (segment (start 121.78 98.77) (end 119.25 101.3) (width 0.8) (layer "B.Cu") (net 10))
 (segment (start 126.6 89.400001) (end 125.560001 89.400001) (width 0.8) (layer "B.Cu") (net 10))
 (segment (start 125.379999 89.400001) (end 125.320498 89.400001) (width 0.8) (layer "B.Cu") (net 10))
 (segment (start 125.33 87.61) (end 125.54 87.4) (width 0.8) (layer "B.Cu") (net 10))
 (segment (start 123.62 88.62) (end 124.84 87.4) (width 0.8) (layer "B.Cu") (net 10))
 (segment (start 127.74 87.4) (end 128.74 87.4) (width 0.8) (layer "B.Cu") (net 10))
 (segment (start 128.74 87.4) (end 128.84 87.3) (width 0.8) (layer "B.Cu") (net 10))
 (segment (start 127.7 87.36) (end 127.74 87.4) (width 0.8) (layer "B.Cu") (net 10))
 (segment (start 125.54 87.4) (end 126.36 87.4) (width 0.8) (layer "B.Cu") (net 10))
 (segment (start 125.3142 89.393703) (end 124.393703 89.393703) (width 0.8) (layer "B.Cu") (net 10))
 (segment (start 127.66 87.4) (end 127.7 87.36) (width 0.8) (layer "B.Cu") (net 10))
 (segment (start 127.81 89.45) (end 127.859999 89.400001) (width 0.8) (layer "B.Cu") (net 10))
 (segment (start 123.62 88.62) (end 123.08 88.62) (width 0.8) (layer "B.Cu") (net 10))
 (segment (start 116.54 87.4) (end 116.64 87.3) (width 0.4) (layer "B.Cu") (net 10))
 (segment (start 126.36 87.4) (end 126.47 87.29) (width 0.8) (layer "B.Cu") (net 10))
 (segment (start 125.560001 89.400001) (end 125.47 89.31) (width 0.8) (layer "B.Cu") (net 10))
 (segment (start 124.84 87.4) (end 125.12 87.4) (width 0.8) (layer "B.Cu") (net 10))
 (segment (start 123.08 88.62) (end 121.76 87.3) (width 0.8) (layer "B.Cu") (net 10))
 (segment (start 126.74 89.43) (end 126.769999 89.400001) (width 0.8) (layer "B.Cu") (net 10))
 (segment (start 126.6 89.400001) (end 126.710001 89.400001) (width 0.8) (layer "B.Cu") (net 10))
 (segment (start 125.47 89.31) (end 125.379999 89.400001) (width 0.8) (layer "B.Cu") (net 10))
 (segment (start 114.7572 87.4) (end 116.54 87.4) (width 0.4) (layer "B.Cu") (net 10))
 (segment (start 126.710001 89.400001) (end 126.74 89.43) (width 0.8) (layer "B.Cu") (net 10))
 (segment (start 125.12 87.4) (end 125.33 87.61) (width 0.8) (layer "B.Cu") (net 10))
 (segment (start 127.760001 89.400001) (end 127.81 89.45) (width 0.8) (layer "B.Cu") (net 10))
 (segment (start 126.58 87.4) (end 126.6 87.4) (width 0.8) (layer "B.Cu") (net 10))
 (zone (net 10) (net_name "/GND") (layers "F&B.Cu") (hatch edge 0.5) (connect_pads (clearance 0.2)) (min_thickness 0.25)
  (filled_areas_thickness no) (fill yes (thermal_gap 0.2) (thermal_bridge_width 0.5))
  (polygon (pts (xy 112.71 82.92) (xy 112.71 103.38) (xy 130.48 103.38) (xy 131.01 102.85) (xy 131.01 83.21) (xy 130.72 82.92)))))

